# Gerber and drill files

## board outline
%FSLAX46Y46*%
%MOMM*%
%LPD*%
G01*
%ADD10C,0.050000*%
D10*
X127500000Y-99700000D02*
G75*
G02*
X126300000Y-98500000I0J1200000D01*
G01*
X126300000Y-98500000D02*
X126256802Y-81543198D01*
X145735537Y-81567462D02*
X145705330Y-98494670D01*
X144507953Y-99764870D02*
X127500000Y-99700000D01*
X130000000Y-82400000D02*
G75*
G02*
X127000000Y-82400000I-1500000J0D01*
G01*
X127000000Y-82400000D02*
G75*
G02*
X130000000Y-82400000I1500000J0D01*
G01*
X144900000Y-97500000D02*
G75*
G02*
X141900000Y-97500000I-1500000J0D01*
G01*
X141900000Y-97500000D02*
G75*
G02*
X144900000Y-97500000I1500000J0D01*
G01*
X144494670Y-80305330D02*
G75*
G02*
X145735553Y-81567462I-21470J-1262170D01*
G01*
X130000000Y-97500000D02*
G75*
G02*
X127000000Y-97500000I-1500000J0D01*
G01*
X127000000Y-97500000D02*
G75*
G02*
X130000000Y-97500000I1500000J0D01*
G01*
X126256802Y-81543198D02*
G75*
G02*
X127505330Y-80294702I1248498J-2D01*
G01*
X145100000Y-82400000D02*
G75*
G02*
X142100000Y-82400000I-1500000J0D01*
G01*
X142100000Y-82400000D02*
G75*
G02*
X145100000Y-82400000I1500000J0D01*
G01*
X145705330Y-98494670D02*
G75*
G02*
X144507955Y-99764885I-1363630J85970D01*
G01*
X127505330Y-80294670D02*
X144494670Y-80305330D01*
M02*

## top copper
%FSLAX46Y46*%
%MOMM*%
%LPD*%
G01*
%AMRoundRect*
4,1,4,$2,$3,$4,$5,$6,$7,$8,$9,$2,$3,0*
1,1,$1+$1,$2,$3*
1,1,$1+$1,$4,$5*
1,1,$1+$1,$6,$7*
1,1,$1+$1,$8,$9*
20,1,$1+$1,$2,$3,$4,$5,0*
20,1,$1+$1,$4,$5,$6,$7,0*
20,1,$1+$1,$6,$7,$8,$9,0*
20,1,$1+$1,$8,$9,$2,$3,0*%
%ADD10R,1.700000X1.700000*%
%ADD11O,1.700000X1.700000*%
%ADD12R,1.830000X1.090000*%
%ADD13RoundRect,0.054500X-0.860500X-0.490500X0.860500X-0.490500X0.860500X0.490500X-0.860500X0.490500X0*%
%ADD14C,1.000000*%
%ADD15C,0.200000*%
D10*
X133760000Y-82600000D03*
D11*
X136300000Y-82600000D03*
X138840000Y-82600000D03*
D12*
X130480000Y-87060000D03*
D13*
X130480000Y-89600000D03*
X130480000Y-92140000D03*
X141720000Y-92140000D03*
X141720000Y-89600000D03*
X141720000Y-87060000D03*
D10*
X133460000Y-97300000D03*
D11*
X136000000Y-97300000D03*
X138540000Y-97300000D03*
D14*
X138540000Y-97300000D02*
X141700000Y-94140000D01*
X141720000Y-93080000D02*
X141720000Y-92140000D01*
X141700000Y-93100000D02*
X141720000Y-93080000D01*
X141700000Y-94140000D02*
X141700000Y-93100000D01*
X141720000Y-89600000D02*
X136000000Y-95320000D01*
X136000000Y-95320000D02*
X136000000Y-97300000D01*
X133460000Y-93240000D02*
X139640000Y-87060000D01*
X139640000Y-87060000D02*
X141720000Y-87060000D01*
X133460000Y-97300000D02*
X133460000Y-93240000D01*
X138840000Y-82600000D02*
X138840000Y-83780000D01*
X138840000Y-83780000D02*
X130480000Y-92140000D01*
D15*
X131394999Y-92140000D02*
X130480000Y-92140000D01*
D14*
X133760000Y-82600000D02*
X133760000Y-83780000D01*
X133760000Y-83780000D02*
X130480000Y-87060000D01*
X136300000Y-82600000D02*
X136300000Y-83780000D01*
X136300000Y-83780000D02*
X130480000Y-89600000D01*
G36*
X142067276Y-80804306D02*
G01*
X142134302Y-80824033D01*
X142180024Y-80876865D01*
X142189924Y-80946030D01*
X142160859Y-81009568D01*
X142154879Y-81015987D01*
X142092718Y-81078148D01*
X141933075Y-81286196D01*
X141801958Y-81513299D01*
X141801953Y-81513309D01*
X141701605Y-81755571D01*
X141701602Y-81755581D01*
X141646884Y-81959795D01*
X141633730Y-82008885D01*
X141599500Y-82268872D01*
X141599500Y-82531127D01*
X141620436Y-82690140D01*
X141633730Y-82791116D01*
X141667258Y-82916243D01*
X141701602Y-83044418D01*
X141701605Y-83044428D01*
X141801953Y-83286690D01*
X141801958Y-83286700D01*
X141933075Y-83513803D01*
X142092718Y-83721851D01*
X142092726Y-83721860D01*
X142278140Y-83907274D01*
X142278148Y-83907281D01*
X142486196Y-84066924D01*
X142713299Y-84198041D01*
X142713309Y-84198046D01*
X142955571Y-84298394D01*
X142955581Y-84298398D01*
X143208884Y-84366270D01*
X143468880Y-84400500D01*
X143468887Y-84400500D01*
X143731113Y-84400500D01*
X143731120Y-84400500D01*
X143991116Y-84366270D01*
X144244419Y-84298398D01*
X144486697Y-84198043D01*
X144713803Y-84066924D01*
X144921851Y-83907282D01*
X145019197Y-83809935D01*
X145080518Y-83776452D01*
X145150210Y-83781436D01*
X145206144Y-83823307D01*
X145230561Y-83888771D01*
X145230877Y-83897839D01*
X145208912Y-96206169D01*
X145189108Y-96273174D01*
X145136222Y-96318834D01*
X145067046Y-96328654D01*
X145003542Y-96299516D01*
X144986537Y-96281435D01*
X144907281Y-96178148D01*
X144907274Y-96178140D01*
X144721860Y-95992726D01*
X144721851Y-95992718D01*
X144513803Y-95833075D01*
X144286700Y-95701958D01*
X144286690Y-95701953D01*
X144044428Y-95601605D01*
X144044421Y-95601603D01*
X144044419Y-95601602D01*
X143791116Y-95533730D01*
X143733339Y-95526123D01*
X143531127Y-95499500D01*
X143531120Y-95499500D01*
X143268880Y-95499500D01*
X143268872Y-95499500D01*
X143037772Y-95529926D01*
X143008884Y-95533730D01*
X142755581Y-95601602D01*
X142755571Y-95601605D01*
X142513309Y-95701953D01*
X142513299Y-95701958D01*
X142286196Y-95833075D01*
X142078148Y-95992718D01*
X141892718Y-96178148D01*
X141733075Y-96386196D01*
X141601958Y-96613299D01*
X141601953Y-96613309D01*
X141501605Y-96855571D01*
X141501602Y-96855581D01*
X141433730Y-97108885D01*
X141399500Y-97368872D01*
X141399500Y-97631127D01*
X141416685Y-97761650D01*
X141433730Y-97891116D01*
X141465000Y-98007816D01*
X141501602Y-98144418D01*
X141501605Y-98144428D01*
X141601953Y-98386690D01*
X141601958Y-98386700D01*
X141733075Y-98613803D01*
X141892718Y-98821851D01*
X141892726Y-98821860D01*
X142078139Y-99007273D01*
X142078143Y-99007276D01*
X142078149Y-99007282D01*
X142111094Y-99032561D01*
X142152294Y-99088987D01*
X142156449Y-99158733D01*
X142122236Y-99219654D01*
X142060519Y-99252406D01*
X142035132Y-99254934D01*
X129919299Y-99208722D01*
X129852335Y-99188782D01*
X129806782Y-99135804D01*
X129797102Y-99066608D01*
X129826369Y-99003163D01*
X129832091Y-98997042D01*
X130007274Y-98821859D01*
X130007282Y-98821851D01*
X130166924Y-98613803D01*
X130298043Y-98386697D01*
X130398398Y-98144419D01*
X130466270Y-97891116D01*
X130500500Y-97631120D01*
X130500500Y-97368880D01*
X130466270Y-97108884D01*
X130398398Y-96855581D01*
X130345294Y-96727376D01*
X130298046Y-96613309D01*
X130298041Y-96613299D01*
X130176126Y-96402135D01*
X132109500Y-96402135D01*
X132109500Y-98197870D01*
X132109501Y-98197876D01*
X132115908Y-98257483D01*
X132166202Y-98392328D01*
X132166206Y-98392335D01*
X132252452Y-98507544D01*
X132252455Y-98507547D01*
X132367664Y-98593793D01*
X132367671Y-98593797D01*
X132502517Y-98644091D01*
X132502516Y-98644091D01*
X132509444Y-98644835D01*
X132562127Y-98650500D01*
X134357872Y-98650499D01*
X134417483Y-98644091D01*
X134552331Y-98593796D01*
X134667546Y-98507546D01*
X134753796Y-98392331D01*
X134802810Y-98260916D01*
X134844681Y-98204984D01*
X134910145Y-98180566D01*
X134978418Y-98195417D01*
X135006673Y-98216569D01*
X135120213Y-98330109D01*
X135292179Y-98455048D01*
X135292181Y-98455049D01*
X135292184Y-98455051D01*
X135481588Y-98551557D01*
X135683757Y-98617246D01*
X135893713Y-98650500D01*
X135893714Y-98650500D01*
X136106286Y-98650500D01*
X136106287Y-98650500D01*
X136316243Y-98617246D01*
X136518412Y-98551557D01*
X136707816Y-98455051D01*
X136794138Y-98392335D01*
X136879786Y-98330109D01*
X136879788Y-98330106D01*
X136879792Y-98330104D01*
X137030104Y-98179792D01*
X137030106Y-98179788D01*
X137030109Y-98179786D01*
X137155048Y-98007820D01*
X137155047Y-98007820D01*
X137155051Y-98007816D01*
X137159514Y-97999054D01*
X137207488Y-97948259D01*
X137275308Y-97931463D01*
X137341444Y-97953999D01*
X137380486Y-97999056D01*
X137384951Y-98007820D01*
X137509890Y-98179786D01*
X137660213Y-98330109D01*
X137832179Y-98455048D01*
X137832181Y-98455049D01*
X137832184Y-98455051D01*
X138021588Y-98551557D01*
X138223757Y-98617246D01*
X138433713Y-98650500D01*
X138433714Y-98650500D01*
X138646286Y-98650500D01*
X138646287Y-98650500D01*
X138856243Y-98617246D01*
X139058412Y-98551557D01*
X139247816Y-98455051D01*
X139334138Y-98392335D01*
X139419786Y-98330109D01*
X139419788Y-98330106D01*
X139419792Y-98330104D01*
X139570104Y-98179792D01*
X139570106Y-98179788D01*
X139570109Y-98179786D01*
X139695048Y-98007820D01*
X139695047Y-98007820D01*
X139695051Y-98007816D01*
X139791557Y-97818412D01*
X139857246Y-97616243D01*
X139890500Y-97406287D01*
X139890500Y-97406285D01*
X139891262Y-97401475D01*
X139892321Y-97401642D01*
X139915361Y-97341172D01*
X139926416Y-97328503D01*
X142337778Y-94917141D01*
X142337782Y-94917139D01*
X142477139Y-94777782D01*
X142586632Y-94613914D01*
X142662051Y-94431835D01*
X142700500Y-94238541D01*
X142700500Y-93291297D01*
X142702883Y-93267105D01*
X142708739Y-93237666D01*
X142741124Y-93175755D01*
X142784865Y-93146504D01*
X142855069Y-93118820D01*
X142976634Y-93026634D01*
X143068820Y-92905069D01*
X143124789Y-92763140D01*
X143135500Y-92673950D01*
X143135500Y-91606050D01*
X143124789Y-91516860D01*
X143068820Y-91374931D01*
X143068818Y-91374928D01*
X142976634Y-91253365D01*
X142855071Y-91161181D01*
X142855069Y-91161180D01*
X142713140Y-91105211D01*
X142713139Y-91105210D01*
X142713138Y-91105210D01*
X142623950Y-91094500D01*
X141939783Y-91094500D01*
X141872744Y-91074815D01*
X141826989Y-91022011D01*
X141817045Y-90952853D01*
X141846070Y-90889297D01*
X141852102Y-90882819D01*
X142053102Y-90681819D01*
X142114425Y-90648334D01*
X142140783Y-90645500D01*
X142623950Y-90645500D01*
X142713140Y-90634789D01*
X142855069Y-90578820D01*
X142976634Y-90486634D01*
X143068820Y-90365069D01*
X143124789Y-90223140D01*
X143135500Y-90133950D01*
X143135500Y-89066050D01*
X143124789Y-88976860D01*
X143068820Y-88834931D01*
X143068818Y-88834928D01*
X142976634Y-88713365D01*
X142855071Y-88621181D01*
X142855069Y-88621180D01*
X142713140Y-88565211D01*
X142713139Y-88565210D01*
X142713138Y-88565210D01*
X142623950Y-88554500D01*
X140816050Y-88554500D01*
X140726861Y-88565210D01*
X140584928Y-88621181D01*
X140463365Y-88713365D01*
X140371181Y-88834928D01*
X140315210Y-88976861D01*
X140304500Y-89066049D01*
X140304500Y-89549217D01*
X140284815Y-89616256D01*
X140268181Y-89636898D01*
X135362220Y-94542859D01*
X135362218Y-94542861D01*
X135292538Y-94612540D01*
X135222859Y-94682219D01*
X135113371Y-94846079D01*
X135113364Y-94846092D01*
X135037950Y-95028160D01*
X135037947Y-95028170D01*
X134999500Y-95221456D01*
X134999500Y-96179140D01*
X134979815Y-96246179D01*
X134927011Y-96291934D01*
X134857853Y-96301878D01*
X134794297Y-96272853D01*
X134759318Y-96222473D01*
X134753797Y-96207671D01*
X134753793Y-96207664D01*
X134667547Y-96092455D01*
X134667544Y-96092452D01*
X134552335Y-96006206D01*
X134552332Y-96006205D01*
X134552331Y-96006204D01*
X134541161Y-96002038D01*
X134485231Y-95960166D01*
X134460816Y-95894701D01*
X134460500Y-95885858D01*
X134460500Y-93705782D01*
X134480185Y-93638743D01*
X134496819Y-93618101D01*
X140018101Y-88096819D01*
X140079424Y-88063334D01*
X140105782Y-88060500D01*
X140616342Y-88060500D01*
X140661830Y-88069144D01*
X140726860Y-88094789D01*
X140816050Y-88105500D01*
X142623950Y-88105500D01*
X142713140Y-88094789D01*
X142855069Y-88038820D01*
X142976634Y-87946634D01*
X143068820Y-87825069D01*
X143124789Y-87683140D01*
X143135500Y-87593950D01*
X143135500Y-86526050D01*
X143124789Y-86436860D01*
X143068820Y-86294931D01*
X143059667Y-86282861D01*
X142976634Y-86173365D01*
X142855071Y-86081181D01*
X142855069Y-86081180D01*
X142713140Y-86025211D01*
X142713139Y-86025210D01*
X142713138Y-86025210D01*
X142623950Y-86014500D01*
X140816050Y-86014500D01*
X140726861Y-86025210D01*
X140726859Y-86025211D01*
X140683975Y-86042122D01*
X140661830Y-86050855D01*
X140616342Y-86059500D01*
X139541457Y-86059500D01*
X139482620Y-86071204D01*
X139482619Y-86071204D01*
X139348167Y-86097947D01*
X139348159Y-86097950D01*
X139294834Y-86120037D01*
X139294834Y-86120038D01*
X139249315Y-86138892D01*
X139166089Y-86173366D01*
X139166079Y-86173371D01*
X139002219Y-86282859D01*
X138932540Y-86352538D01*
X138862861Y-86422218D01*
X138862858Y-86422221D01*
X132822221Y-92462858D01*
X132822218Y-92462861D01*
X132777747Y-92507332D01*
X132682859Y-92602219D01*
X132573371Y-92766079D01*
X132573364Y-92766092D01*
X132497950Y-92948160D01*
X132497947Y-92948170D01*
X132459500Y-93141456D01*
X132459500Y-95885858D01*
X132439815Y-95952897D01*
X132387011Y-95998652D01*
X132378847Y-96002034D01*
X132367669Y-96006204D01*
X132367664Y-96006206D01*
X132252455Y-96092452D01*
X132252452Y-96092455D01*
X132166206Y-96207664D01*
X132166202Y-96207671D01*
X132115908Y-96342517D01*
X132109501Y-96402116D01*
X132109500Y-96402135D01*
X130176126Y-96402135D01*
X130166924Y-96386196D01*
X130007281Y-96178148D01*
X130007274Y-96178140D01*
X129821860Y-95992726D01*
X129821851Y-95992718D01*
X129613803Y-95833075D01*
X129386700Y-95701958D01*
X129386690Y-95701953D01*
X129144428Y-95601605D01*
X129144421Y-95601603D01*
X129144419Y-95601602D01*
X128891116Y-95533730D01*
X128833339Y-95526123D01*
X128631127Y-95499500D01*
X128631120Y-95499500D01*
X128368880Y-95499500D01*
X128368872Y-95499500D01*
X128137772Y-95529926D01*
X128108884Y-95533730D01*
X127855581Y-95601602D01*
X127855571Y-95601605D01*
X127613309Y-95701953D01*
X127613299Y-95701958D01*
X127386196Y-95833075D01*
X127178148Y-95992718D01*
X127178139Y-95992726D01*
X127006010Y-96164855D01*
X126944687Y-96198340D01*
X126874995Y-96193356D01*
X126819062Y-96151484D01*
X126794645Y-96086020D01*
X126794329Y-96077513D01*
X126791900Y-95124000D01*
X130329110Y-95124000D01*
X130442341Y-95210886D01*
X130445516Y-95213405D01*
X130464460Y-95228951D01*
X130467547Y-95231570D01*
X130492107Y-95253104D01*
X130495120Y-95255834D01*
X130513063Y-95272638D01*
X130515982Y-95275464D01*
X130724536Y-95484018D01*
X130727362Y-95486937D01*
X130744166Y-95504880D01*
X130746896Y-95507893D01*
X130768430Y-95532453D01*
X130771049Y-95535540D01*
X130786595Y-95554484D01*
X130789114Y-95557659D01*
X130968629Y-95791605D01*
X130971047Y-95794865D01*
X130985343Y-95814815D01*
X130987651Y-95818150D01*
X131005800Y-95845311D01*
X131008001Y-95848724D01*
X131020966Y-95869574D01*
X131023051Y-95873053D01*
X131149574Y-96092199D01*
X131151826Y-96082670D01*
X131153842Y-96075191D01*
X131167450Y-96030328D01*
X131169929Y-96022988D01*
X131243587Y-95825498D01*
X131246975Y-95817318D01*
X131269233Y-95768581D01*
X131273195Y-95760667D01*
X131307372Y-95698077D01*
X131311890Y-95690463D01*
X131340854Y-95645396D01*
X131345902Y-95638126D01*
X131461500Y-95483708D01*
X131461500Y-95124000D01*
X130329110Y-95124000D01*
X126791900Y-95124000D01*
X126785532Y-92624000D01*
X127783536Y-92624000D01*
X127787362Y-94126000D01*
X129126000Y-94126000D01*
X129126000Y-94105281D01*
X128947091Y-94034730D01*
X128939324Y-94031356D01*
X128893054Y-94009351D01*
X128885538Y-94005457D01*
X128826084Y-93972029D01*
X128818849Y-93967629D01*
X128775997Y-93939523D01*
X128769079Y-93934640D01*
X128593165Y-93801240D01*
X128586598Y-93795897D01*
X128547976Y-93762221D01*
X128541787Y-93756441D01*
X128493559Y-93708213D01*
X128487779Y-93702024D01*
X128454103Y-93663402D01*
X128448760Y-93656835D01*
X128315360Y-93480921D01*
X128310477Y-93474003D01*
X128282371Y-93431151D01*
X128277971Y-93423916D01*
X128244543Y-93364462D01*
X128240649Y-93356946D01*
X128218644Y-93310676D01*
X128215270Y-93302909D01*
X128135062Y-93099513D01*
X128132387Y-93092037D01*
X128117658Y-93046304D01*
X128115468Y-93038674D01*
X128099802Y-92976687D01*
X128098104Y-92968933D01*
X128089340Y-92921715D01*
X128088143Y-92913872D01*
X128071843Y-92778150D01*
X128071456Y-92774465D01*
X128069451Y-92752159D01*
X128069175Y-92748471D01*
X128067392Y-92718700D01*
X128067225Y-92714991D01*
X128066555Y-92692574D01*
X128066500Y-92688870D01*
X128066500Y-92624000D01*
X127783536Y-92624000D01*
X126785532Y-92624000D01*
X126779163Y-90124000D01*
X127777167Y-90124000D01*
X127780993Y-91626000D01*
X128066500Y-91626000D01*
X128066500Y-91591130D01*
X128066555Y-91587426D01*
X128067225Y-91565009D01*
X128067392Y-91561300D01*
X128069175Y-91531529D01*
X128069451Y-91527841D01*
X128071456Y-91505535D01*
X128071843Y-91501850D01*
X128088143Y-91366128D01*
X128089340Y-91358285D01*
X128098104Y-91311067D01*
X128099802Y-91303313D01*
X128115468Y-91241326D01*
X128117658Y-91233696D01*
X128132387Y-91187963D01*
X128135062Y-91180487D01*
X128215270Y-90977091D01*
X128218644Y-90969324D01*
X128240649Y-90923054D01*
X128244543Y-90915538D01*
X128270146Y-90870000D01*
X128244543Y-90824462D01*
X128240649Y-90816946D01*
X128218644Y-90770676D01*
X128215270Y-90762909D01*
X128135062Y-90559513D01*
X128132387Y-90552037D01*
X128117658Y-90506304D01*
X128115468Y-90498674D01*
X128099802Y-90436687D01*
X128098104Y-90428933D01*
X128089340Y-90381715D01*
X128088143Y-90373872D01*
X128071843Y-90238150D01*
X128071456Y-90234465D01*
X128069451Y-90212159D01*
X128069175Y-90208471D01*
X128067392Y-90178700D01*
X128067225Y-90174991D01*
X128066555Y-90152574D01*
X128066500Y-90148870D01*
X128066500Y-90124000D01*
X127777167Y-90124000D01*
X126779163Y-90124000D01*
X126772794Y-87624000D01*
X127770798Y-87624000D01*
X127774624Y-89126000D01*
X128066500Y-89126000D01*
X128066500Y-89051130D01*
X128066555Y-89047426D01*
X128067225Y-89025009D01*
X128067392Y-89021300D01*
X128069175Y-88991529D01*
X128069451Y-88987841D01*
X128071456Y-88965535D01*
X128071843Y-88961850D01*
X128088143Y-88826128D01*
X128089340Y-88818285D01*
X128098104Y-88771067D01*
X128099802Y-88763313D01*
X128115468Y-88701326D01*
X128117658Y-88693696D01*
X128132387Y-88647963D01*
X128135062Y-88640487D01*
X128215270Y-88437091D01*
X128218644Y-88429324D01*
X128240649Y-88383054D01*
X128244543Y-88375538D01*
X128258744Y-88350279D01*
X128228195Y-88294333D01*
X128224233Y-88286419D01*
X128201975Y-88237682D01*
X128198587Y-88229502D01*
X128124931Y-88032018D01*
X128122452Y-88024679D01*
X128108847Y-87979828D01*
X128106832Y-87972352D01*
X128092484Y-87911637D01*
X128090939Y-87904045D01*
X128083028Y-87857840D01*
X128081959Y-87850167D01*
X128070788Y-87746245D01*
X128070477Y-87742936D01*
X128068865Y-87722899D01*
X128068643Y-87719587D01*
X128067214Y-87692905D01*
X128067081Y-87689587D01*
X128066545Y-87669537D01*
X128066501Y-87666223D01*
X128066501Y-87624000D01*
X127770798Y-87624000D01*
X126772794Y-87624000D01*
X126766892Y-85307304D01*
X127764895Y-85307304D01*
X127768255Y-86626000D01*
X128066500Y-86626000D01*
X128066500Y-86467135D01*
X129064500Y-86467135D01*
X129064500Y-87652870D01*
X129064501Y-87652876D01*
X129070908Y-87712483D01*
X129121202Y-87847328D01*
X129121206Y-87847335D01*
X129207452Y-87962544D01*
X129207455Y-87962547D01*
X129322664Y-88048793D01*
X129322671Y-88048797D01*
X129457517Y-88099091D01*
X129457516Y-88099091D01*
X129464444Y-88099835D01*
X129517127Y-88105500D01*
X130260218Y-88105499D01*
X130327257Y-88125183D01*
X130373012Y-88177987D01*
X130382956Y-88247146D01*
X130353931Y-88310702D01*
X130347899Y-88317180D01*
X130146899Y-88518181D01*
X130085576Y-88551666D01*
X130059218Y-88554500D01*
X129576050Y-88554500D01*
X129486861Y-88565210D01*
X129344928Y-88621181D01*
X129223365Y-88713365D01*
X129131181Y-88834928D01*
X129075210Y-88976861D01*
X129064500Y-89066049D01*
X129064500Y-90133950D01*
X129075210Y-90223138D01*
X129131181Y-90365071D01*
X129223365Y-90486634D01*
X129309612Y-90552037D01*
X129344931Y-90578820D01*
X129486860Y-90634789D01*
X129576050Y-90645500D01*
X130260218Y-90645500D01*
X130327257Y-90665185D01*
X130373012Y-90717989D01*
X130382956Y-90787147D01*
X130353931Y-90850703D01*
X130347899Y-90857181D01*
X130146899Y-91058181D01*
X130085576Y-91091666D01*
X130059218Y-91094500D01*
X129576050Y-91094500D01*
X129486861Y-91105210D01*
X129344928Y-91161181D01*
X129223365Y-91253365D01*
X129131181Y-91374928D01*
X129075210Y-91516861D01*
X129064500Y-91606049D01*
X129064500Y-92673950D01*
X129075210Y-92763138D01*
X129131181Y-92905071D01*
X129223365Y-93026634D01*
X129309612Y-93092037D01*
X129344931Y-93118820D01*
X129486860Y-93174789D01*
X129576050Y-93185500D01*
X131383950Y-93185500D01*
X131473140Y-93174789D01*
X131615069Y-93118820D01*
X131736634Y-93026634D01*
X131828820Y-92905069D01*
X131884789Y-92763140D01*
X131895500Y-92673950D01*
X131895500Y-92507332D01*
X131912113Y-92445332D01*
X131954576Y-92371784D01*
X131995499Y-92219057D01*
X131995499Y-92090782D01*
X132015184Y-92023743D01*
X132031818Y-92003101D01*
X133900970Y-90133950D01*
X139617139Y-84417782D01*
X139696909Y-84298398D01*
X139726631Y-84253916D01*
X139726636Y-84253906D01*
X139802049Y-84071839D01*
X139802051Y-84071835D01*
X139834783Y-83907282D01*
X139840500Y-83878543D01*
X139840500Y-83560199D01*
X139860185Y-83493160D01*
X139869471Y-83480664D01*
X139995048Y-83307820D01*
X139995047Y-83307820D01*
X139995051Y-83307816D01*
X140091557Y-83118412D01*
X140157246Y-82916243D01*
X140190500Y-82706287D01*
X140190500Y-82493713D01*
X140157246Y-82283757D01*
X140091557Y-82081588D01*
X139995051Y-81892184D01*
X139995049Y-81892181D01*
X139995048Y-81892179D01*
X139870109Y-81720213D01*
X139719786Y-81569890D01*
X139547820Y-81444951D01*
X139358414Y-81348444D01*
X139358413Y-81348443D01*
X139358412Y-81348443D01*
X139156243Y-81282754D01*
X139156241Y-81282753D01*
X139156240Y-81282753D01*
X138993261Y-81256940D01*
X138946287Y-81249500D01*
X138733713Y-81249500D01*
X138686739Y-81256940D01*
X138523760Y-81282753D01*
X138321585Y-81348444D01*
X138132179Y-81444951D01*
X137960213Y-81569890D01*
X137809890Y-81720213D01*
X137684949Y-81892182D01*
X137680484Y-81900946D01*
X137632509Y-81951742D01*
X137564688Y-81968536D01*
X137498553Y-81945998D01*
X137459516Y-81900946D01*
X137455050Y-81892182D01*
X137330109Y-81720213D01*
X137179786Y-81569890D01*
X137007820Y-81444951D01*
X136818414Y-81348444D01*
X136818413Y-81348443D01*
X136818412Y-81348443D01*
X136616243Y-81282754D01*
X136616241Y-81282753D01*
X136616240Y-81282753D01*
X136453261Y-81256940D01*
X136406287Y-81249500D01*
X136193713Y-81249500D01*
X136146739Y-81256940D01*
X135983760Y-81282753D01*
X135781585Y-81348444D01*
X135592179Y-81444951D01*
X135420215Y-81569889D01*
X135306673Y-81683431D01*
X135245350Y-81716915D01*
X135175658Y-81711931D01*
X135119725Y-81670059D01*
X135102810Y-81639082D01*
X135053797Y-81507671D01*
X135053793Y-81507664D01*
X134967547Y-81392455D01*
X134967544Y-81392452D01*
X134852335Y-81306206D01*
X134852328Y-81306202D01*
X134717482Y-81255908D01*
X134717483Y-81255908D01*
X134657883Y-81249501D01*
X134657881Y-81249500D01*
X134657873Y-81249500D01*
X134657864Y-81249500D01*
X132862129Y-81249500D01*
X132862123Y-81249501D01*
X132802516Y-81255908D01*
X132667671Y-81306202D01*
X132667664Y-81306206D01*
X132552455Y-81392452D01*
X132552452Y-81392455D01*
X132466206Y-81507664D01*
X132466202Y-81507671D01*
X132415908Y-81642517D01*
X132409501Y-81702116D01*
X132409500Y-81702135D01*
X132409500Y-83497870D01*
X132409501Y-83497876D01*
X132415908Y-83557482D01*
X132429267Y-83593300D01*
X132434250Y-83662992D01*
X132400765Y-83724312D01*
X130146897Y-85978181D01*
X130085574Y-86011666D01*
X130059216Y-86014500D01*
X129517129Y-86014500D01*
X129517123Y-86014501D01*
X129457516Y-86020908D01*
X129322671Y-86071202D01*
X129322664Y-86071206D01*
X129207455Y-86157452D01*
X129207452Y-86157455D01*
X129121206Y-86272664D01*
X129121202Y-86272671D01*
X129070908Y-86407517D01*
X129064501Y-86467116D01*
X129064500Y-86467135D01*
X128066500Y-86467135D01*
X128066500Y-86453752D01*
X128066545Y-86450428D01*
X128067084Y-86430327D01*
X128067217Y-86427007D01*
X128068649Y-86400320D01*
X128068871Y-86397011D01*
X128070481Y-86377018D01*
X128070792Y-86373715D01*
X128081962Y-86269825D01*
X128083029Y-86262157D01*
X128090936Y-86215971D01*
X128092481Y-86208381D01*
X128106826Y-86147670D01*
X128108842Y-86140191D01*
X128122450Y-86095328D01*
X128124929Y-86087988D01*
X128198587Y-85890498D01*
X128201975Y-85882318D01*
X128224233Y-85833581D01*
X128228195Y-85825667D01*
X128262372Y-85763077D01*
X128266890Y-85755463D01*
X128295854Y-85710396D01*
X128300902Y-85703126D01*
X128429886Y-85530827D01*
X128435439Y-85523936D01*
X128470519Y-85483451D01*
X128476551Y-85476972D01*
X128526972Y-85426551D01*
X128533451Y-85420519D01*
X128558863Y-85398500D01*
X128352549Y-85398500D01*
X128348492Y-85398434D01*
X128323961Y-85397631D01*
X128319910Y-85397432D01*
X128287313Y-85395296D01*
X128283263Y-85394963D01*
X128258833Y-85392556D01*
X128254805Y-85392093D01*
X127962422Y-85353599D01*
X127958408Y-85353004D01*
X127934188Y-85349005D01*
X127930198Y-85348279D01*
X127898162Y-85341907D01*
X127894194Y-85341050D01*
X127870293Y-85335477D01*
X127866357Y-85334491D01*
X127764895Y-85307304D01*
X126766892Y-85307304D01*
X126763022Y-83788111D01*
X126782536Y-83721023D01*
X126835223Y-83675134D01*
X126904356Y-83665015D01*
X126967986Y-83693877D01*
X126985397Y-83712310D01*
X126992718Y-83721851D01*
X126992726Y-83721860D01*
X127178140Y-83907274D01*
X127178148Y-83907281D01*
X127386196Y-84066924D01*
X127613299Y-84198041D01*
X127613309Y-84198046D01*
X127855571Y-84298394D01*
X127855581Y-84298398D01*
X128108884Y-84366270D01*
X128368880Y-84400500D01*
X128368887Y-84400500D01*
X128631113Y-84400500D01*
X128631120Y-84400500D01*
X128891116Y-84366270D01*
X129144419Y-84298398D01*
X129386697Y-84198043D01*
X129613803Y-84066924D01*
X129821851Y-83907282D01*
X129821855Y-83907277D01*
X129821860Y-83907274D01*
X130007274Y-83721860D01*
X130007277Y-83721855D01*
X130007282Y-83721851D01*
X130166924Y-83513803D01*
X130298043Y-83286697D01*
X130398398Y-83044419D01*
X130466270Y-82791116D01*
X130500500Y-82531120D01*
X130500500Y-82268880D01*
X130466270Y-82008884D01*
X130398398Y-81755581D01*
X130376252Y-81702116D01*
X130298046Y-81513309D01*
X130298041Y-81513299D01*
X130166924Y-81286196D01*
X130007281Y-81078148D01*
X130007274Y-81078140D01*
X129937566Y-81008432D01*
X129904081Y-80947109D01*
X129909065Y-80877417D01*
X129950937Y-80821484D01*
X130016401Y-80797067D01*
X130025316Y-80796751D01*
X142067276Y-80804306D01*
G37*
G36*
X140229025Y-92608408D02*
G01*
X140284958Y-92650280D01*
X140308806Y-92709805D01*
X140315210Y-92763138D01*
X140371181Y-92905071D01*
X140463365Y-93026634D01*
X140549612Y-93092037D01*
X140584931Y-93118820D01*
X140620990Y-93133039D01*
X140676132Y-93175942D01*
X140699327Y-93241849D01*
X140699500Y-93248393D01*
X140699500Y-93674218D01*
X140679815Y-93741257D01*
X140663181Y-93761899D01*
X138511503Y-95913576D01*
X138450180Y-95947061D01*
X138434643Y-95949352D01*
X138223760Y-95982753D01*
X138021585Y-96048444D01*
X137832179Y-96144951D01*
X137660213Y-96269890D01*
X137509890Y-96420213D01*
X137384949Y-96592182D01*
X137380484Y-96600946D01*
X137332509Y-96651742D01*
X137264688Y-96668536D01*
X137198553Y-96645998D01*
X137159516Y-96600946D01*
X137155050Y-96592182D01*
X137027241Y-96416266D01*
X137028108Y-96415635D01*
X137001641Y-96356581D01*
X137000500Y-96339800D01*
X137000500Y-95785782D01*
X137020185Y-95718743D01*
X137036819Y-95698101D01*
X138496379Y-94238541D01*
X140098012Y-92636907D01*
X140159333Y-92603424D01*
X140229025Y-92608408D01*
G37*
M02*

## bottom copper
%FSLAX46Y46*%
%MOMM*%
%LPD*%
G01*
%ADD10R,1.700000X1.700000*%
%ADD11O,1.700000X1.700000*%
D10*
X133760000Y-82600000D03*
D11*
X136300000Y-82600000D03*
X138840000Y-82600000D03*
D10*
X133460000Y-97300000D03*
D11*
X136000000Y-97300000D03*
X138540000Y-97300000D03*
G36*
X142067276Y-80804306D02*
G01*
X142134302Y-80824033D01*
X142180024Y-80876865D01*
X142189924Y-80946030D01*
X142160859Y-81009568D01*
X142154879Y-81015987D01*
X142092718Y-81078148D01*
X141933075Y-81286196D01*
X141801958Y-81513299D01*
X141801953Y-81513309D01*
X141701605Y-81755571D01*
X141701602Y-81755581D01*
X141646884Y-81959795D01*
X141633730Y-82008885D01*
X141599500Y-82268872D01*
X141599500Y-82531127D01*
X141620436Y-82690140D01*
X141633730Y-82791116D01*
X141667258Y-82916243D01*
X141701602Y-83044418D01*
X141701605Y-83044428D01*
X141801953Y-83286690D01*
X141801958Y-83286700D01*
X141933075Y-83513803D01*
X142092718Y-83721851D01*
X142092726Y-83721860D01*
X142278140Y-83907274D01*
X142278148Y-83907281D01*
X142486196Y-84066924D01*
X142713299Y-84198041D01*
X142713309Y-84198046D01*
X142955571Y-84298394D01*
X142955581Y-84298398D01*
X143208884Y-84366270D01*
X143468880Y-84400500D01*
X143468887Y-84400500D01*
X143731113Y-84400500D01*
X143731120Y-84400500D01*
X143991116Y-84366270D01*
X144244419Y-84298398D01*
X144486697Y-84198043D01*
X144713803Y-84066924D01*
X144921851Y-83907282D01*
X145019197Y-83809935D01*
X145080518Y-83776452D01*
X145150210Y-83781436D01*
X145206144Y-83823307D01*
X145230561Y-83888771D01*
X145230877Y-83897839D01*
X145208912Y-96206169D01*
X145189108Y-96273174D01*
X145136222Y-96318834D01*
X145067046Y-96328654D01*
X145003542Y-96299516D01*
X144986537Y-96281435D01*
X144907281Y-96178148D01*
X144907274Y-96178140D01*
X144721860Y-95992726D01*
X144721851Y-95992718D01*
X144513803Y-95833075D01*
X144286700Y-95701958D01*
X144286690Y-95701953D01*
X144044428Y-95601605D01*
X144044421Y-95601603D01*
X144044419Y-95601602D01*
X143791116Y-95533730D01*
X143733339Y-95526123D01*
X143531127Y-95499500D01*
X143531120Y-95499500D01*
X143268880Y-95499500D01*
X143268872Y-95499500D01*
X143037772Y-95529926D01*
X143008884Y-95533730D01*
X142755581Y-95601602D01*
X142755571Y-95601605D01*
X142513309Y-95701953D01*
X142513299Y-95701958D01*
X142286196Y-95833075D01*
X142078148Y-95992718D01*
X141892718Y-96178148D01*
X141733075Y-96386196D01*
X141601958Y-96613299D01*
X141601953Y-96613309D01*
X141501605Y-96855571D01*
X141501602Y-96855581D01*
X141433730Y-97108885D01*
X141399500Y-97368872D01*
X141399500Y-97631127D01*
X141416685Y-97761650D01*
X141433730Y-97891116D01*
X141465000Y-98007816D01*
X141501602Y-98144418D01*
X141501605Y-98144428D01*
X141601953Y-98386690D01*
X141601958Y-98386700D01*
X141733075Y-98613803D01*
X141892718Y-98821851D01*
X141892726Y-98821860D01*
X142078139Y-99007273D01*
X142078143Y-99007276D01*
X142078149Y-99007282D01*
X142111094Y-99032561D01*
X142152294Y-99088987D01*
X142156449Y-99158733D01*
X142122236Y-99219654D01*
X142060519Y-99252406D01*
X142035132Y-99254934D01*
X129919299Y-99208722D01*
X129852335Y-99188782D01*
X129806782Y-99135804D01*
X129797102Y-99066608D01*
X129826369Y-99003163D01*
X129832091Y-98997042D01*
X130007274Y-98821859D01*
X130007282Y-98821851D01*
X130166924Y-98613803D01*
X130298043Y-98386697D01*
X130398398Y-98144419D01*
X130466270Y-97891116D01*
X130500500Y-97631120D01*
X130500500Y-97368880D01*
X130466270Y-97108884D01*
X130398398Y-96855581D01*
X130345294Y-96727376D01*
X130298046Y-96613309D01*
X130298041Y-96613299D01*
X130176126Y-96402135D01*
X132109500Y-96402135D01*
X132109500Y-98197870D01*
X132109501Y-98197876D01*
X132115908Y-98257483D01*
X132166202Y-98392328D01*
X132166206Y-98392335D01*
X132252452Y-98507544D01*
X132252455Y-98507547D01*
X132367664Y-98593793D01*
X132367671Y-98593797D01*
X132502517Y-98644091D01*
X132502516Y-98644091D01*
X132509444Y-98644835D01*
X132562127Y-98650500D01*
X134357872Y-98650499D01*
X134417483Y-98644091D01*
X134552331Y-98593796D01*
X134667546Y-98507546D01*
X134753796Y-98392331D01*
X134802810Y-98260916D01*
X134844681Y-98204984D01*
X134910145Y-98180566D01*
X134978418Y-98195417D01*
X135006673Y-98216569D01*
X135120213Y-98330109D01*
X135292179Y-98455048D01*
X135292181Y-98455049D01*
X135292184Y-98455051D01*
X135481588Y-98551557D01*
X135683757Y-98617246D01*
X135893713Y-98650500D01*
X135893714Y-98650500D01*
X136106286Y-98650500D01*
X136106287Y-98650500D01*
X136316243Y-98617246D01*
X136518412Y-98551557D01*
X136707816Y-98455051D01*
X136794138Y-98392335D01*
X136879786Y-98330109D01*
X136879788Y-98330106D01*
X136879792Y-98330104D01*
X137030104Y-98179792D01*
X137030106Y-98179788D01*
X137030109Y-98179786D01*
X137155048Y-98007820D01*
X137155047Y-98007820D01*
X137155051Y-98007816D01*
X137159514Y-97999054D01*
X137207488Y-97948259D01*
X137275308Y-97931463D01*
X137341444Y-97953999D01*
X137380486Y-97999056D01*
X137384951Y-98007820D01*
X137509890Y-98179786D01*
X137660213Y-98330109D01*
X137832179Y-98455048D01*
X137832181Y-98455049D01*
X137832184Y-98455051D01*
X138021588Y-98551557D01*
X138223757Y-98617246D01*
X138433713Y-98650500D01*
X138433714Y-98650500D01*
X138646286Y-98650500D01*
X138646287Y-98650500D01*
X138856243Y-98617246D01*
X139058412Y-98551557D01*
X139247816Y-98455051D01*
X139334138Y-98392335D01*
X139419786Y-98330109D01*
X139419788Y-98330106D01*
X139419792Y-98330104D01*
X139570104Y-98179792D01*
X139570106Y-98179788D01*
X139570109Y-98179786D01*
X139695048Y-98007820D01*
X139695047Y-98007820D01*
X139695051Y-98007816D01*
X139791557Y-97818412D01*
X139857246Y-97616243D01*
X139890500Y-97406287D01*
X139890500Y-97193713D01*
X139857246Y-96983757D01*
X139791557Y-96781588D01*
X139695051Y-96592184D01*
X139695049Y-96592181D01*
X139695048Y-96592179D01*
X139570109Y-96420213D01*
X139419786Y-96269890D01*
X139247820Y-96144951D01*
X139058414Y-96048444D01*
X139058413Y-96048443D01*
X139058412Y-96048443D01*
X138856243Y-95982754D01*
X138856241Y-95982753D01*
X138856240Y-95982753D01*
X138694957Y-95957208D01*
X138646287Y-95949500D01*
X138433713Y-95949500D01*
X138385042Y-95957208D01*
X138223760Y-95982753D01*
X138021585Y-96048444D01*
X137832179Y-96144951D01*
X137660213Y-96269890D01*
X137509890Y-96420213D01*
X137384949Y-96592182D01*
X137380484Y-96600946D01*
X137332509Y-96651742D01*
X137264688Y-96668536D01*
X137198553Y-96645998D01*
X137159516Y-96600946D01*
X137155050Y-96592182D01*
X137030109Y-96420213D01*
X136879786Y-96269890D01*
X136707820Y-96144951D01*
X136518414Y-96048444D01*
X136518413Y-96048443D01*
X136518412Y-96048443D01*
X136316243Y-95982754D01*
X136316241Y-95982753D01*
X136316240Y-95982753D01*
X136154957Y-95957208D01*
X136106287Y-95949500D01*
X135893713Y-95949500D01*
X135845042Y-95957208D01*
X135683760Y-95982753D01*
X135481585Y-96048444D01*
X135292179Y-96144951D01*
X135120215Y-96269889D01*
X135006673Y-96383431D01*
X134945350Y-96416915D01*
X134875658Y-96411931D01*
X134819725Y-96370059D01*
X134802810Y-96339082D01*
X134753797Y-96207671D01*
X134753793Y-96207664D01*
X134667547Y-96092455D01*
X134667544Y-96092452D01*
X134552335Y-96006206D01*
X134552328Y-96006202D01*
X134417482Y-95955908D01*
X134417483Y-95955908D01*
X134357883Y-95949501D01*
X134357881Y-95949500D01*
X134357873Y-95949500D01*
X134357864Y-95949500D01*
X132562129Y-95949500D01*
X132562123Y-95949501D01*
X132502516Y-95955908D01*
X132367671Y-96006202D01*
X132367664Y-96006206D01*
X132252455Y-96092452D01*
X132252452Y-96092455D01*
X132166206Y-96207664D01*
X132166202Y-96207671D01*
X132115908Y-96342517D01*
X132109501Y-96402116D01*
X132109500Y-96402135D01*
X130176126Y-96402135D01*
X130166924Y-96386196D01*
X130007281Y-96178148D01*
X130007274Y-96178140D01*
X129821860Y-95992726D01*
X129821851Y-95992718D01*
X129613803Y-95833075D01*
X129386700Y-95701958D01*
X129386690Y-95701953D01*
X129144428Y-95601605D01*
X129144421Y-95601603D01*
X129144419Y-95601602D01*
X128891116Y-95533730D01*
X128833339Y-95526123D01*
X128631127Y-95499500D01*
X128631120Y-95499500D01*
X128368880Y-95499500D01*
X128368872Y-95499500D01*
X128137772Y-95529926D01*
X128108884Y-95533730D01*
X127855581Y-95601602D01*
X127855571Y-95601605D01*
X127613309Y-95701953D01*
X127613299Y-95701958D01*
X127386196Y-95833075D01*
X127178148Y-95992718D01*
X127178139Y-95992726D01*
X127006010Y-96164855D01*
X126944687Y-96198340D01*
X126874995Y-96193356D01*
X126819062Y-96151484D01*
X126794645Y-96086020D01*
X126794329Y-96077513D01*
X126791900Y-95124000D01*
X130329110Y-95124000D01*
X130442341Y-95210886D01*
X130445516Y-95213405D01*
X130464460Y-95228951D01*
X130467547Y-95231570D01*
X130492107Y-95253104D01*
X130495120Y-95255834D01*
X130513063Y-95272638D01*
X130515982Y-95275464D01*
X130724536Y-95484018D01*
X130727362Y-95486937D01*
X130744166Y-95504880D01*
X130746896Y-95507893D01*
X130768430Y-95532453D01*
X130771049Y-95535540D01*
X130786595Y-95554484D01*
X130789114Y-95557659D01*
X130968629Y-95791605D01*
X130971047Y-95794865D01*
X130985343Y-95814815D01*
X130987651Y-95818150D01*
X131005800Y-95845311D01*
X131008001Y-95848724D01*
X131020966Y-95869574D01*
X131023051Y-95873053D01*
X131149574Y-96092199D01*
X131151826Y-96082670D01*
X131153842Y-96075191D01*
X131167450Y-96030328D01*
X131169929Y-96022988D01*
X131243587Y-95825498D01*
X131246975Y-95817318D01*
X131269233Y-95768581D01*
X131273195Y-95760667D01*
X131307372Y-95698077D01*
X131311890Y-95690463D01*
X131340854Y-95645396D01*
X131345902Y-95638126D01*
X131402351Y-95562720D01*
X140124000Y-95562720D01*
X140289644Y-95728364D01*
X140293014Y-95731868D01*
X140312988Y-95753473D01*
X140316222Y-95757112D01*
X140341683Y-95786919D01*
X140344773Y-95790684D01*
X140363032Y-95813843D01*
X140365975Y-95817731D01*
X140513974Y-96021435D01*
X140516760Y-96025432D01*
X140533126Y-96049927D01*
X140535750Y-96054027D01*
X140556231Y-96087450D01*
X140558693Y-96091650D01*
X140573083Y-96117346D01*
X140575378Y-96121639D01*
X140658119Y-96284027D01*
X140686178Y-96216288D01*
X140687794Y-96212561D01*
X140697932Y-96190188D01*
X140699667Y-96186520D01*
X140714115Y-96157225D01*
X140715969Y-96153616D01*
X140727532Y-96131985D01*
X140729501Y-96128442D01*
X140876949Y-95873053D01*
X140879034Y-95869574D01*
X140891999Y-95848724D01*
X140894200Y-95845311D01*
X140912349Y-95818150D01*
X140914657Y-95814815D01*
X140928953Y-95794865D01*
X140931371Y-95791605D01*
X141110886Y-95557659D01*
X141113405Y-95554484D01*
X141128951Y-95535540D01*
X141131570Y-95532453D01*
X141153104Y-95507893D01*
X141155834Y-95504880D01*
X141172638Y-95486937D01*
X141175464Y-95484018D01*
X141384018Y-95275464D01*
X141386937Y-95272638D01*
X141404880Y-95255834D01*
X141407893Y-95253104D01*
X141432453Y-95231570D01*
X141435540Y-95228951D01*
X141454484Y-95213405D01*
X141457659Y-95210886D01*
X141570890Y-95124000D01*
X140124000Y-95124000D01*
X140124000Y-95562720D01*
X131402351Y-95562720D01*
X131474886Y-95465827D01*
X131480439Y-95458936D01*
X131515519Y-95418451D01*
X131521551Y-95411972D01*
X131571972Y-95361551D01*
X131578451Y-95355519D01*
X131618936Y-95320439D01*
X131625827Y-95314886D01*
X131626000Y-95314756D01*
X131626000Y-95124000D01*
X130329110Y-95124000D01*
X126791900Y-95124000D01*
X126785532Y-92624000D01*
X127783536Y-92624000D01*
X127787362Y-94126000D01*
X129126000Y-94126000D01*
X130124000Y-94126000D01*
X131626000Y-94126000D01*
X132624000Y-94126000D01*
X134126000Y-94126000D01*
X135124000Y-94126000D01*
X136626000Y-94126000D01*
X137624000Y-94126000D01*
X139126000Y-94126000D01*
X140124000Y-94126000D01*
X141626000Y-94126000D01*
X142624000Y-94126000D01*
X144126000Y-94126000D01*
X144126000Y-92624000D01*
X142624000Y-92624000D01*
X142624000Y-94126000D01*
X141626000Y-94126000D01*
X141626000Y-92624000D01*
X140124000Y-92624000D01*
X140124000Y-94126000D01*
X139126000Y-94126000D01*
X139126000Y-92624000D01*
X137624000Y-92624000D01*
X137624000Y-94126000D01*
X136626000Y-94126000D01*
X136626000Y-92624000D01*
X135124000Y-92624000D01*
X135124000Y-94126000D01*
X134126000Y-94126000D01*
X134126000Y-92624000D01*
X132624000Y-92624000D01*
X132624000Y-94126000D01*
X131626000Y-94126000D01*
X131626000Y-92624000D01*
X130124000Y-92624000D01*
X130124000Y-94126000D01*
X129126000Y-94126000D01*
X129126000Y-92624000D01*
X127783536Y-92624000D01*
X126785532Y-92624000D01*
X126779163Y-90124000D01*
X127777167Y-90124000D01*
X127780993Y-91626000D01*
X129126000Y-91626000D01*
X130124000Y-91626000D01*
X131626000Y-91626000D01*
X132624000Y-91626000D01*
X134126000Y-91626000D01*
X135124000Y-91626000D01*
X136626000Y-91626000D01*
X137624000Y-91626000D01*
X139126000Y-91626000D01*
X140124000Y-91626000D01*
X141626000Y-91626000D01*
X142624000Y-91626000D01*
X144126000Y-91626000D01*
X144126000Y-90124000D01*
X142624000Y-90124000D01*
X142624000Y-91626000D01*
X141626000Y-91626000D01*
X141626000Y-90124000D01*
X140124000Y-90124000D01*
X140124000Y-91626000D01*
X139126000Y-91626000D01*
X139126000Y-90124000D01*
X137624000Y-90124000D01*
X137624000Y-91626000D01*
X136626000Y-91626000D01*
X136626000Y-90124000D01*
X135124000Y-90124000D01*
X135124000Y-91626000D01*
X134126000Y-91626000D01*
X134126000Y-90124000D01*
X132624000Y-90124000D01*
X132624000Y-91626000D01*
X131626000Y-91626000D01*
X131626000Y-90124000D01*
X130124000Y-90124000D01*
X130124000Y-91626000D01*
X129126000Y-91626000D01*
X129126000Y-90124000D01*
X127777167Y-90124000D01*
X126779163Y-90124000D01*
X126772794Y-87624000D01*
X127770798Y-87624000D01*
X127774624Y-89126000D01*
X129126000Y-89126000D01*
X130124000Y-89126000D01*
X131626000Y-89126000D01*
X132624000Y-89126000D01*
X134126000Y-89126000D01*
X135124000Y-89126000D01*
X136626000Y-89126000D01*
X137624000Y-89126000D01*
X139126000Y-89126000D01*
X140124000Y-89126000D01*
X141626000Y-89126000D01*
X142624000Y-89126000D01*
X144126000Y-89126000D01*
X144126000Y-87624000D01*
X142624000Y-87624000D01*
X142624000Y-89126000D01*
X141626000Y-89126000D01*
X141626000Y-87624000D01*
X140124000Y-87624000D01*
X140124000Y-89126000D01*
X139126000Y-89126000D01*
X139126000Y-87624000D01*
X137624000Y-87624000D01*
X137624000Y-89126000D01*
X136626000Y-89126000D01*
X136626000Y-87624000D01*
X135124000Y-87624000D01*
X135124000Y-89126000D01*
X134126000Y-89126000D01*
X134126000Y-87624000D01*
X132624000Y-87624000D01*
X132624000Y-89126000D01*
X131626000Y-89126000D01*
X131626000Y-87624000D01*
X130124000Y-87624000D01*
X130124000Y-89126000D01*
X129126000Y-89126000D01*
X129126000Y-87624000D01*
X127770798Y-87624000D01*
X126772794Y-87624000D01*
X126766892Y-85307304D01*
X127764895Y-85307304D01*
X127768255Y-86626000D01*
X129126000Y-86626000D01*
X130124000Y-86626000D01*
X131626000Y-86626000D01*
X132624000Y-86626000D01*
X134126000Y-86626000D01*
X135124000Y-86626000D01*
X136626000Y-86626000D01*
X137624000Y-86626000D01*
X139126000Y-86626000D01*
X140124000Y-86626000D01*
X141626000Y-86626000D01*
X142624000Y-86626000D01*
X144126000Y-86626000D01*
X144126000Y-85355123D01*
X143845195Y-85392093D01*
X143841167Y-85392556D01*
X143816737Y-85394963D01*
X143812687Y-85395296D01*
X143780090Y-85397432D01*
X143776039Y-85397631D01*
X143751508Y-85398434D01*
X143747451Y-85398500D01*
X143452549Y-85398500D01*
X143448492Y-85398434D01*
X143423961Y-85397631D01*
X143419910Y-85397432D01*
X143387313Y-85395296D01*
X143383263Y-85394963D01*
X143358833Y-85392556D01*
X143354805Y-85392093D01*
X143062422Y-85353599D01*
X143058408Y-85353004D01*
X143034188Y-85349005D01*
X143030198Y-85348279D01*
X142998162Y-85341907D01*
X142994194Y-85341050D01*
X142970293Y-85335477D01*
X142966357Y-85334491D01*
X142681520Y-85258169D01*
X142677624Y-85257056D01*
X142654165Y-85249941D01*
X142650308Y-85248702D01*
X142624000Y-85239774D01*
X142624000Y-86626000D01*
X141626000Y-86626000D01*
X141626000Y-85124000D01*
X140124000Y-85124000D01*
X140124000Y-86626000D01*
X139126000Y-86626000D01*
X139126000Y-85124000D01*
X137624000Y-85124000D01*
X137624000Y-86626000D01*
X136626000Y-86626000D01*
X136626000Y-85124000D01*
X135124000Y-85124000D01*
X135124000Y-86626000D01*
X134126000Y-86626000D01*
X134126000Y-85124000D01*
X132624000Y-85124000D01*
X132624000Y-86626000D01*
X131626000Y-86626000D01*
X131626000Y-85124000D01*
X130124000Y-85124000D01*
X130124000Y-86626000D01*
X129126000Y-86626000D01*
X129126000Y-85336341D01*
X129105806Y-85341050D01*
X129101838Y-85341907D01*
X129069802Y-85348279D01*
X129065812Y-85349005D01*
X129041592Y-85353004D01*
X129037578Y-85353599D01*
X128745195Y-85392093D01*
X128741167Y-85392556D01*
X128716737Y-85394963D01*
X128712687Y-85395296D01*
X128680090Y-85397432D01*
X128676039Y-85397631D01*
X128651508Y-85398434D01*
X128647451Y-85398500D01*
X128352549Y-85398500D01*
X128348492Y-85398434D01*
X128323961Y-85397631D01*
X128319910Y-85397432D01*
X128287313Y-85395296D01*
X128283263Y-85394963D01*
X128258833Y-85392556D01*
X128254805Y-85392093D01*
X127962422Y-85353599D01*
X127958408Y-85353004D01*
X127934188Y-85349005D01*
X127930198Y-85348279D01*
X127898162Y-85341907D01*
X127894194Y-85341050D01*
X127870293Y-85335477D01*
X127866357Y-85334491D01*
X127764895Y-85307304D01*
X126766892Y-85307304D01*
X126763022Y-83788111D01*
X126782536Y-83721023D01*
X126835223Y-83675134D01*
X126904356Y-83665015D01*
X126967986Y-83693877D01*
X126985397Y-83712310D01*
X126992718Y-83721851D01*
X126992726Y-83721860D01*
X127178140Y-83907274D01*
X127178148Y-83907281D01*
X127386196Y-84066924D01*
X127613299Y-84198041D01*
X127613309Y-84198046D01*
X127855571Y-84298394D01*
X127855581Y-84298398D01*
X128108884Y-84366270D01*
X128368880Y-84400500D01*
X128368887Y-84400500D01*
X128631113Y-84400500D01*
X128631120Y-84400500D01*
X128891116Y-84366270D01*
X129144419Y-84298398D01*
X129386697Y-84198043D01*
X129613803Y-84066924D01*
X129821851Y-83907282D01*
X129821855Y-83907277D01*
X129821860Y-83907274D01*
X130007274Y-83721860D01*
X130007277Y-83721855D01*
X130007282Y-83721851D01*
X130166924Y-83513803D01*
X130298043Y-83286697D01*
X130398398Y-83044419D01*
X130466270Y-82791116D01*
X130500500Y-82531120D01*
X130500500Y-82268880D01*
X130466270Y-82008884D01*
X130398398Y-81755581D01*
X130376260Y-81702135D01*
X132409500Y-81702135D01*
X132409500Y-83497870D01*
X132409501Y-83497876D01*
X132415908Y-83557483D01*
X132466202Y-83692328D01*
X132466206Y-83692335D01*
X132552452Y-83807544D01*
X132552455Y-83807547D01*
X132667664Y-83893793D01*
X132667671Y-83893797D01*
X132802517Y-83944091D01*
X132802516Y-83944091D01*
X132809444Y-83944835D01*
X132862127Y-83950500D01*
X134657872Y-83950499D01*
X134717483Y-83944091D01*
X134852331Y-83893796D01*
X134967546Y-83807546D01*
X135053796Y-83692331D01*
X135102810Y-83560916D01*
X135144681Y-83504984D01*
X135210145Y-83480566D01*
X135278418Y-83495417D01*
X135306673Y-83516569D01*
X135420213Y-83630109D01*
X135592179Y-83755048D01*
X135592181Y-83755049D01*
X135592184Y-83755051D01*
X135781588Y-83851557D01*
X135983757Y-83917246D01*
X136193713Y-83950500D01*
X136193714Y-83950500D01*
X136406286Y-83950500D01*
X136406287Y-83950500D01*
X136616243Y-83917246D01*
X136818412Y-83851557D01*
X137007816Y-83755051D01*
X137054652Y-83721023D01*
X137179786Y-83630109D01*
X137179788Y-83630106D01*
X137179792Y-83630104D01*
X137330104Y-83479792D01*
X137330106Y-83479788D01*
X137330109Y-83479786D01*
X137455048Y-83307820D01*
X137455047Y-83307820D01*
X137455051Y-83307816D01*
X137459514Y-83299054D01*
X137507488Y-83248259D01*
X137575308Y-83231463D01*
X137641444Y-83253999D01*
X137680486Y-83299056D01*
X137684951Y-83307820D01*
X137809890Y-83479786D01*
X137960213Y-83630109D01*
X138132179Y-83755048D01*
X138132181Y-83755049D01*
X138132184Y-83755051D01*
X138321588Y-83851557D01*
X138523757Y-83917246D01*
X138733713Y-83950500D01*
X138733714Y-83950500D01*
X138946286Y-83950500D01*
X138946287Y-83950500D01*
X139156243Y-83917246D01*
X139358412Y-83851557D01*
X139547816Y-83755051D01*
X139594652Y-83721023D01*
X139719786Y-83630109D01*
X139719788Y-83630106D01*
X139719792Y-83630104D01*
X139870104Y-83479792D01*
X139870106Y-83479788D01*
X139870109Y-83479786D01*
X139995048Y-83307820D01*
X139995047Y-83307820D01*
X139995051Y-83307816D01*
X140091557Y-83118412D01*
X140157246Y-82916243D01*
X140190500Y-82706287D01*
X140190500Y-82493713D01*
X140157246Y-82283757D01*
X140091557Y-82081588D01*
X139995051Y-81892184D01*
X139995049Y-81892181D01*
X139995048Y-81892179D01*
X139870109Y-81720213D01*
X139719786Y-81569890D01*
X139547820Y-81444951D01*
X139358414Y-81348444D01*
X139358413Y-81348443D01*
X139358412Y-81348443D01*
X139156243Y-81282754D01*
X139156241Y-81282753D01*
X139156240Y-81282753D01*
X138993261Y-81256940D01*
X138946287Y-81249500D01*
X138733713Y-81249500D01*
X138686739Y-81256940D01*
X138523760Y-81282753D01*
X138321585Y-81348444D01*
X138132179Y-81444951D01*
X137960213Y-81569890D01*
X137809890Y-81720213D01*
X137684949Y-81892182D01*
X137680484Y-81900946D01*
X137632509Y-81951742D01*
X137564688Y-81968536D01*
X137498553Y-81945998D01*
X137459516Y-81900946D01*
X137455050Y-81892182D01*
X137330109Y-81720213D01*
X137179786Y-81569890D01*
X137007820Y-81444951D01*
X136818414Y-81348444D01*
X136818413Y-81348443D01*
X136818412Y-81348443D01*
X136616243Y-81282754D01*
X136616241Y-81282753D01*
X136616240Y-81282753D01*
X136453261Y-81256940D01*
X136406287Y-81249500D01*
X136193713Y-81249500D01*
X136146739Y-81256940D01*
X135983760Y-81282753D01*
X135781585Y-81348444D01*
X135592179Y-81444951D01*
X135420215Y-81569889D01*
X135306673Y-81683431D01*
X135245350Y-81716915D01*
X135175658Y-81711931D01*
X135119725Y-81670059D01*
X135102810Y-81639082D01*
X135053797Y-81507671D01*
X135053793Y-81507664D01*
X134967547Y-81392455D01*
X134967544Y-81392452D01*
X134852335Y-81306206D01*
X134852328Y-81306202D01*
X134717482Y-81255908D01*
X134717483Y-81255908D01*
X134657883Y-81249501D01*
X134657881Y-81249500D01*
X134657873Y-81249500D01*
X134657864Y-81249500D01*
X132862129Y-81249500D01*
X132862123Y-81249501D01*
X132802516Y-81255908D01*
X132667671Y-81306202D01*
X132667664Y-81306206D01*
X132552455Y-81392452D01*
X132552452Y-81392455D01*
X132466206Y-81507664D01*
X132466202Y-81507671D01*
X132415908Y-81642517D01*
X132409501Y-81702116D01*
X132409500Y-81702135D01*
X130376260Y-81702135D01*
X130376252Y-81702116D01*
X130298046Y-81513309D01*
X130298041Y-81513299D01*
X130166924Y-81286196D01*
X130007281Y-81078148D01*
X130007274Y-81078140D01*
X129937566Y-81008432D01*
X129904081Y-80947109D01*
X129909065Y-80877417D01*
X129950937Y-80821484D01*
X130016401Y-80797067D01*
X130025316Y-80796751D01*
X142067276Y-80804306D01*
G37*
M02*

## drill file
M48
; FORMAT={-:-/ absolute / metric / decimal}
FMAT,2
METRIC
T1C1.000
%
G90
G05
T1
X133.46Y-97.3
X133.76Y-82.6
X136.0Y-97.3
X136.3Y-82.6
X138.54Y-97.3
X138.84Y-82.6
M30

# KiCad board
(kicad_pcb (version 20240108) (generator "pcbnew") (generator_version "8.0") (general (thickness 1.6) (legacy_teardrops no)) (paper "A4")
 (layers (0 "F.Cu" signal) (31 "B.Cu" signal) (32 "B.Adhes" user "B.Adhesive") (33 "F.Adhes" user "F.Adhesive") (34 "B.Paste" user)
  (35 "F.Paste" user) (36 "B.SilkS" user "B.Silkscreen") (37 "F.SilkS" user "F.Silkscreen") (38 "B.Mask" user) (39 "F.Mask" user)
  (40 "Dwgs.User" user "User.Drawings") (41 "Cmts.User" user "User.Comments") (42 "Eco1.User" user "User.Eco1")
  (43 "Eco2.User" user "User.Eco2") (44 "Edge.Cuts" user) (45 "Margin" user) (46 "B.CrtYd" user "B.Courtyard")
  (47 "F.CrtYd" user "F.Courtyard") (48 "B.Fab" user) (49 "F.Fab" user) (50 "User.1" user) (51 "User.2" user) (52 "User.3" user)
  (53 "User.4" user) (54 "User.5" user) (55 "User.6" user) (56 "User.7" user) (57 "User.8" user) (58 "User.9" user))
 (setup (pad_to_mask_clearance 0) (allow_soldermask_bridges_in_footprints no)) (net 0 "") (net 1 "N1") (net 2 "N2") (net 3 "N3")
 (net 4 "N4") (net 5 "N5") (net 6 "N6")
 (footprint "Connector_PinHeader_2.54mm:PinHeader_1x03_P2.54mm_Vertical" (layer "F.Cu") (at 133.76 82.6 90)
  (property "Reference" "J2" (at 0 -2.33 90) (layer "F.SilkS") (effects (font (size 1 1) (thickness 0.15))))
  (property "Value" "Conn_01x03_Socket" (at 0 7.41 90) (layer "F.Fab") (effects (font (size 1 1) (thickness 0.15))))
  (pad "1" thru_hole rect (at 0 0 90) (size 1.7 1.7) (drill 1) (layers "*.Cu" "*.Mask") (remove_unused_layers no) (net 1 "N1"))
  (pad "2" thru_hole oval (at 0 2.54 90) (size 1.7 1.7) (drill 1) (layers "*.Cu" "*.Mask") (remove_unused_layers no) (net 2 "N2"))
  (pad "3" thru_hole oval (at 0 5.08 90) (size 1.7 1.7) (drill 1) (layers "*.Cu" "*.Mask") (remove_unused_layers no) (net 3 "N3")))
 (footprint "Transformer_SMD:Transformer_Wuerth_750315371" (layer "F.Cu") (at 136.1 89.6)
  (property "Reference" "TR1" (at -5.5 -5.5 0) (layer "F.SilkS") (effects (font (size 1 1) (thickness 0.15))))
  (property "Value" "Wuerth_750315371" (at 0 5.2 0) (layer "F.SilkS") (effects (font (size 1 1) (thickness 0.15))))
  (pad "1" smd rect (at -5.62 -2.54) (size 1.83 1.09) (layers "F.Cu" "F.Paste" "F.Mask") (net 1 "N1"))
  (pad "2" smd roundrect (at -5.62 0) (size 1.83 1.09) (layers "F.Cu" "F.Paste" "F.Mask") (roundrect_rratio 0.05) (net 2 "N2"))
  (pad "3" smd roundrect (at -5.62 2.54) (size 1.83 1.09) (layers "F.Cu" "F.Paste" "F.Mask") (roundrect_rratio 0.05) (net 3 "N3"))
  (pad "4" smd roundrect (at 5.62 2.54) (size 1.83 1.09) (layers "F.Cu" "F.Paste" "F.Mask") (roundrect_rratio 0.05) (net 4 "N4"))
  (pad "5" smd roundrect (at 5.62 0) (size 1.83 1.09) (layers "F.Cu" "F.Paste" "F.Mask") (roundrect_rratio 0.05) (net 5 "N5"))
  (pad "6" smd roundrect (at 5.62 -2.54) (size 1.83 1.09) (layers "F.Cu" "F.Paste" "F.Mask") (roundrect_rratio 0.05) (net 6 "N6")))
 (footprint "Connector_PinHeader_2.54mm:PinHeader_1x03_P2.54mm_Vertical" (layer "F.Cu") (at 133.46 97.3 90)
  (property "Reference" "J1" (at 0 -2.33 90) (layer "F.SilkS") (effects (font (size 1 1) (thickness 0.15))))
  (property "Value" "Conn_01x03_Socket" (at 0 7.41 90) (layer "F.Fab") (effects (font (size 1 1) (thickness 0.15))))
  (pad "1" thru_hole rect (at 0 0 90) (size 1.7 1.7) (drill 1) (layers "*.Cu" "*.Mask") (remove_unused_layers no) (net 6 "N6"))
  (pad "2" thru_hole oval (at 0 2.54 90) (size 1.7 1.7) (drill 1) (layers "*.Cu" "*.Mask") (remove_unused_layers no) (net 5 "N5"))
  (pad "3" thru_hole oval (at 0 5.08 90) (size 1.7 1.7) (drill 1) (layers "*.Cu" "*.Mask") (remove_unused_layers no) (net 4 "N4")))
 (gr_arc (start 127.5 99.7) (mid 126.651472 99.348528) (end 126.3 98.5) (stroke (width 0.05) (type default)) (layer "Edge.Cuts"))
 (gr_line (start 126.3 98.5) (end 126.256802 81.543198) (stroke (width 0.05) (type default)) (layer "Edge.Cuts"))
 (gr_line (start 145.735537 81.567462) (end 145.70533 98.49467) (stroke (width 0.05) (type default)) (layer "Edge.Cuts"))
 (gr_line (start 144.507953 99.76487) (end 127.5 99.7) (stroke (width 0.05) (type default)) (layer "Edge.Cuts"))
 (gr_circle (center 128.5 82.4) (end 130 82.4) (stroke (width 0.05) (type default)) (fill none) (layer "Edge.Cuts"))
 (gr_circle (center 143.4 97.5) (end 144.9 97.5) (stroke (width 0.05) (type default)) (fill none) (layer "Edge.Cuts"))
 (gr_arc (start 144.49467 80.30533) (mid 145.373365 80.682486) (end 145.735537 81.567462) (stroke (width 0.05) (type default))
  (layer "Edge.Cuts"))
 (gr_circle (center 128.5 97.5) (end 130 97.5) (stroke (width 0.05) (type default)) (fill none) (layer "Edge.Cuts"))
 (gr_arc (start 126.256802 81.543198) (mid 126.622487 80.660355) (end 127.50533 80.29467) (stroke (width 0.05) (type default))
  (layer "Edge.Cuts"))
 (gr_circle (center 143.6 82.4) (end 145.1 82.4) (stroke (width 0.05) (type default)) (fill none) (layer "Edge.Cuts"))
 (gr_arc (start 145.70533 98.49467) (mid 145.335923 99.345906) (end 144.507953 99.76487) (stroke (width 0.05) (type default))
  (layer "Edge.Cuts"))
 (gr_line (start 127.50533 80.29467) (end 144.49467 80.30533) (stroke (width 0.05) (type default)) (layer "Edge.Cuts"))
 (segment (start 138.54 97.3) (end 141.7 94.14) (width 1) (layer "F.Cu") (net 4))
 (segment (start 141.72 93.08) (end 141.72 92.14) (width 1) (layer "F.Cu") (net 4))
 (segment (start 141.7 93.1) (end 141.72 93.08) (width 1) (layer "F.Cu") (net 4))
 (segment (start 141.7 94.14) (end 141.7 93.1) (width 1) (layer "F.Cu") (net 4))
 (segment (start 141.72 89.6) (end 136 95.32) (width 1) (layer "F.Cu") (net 5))
 (segment (start 136 95.32) (end 136 97.3) (width 1) (layer "F.Cu") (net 5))
 (segment (start 133.46 93.24) (end 139.64 87.06) (width 1) (layer "F.Cu") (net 6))
 (segment (start 139.64 87.06) (end 141.72 87.06) (width 1) (layer "F.Cu") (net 6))
 (segment (start 133.46 97.3) (end 133.46 93.24) (width 1) (layer "F.Cu") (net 6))
 (segment (start 138.84 82.6) (end 138.84 83.78) (width 1) (layer "F.Cu") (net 3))
 (segment (start 138.84 83.78) (end 130.48 92.14) (width 1) (layer "F.Cu") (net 3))
 (segment (start 131.394999 92.14) (end 130.48 92.14) (width 0.2) (layer "F.Cu") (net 3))
 (segment (start 133.76 82.6) (end 133.76 83.78) (width 1) (layer "F.Cu") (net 1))
 (segment (start 133.76 83.78) (end 130.48 87.06) (width 1) (layer "F.Cu") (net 1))
 (segment (start 136.3 82.6) (end 136.3 83.78) (width 1) (layer "F.Cu") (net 2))
 (segment (start 136.3 83.78) (end 130.48 89.6) (width 1) (layer "F.Cu") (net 2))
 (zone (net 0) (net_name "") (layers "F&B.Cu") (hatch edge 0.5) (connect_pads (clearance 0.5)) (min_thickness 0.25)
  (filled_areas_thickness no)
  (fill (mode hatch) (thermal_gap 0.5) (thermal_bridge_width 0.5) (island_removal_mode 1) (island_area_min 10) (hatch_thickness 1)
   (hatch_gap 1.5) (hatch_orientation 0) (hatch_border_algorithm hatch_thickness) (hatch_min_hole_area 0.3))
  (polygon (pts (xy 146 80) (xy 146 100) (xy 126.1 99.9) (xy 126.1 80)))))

